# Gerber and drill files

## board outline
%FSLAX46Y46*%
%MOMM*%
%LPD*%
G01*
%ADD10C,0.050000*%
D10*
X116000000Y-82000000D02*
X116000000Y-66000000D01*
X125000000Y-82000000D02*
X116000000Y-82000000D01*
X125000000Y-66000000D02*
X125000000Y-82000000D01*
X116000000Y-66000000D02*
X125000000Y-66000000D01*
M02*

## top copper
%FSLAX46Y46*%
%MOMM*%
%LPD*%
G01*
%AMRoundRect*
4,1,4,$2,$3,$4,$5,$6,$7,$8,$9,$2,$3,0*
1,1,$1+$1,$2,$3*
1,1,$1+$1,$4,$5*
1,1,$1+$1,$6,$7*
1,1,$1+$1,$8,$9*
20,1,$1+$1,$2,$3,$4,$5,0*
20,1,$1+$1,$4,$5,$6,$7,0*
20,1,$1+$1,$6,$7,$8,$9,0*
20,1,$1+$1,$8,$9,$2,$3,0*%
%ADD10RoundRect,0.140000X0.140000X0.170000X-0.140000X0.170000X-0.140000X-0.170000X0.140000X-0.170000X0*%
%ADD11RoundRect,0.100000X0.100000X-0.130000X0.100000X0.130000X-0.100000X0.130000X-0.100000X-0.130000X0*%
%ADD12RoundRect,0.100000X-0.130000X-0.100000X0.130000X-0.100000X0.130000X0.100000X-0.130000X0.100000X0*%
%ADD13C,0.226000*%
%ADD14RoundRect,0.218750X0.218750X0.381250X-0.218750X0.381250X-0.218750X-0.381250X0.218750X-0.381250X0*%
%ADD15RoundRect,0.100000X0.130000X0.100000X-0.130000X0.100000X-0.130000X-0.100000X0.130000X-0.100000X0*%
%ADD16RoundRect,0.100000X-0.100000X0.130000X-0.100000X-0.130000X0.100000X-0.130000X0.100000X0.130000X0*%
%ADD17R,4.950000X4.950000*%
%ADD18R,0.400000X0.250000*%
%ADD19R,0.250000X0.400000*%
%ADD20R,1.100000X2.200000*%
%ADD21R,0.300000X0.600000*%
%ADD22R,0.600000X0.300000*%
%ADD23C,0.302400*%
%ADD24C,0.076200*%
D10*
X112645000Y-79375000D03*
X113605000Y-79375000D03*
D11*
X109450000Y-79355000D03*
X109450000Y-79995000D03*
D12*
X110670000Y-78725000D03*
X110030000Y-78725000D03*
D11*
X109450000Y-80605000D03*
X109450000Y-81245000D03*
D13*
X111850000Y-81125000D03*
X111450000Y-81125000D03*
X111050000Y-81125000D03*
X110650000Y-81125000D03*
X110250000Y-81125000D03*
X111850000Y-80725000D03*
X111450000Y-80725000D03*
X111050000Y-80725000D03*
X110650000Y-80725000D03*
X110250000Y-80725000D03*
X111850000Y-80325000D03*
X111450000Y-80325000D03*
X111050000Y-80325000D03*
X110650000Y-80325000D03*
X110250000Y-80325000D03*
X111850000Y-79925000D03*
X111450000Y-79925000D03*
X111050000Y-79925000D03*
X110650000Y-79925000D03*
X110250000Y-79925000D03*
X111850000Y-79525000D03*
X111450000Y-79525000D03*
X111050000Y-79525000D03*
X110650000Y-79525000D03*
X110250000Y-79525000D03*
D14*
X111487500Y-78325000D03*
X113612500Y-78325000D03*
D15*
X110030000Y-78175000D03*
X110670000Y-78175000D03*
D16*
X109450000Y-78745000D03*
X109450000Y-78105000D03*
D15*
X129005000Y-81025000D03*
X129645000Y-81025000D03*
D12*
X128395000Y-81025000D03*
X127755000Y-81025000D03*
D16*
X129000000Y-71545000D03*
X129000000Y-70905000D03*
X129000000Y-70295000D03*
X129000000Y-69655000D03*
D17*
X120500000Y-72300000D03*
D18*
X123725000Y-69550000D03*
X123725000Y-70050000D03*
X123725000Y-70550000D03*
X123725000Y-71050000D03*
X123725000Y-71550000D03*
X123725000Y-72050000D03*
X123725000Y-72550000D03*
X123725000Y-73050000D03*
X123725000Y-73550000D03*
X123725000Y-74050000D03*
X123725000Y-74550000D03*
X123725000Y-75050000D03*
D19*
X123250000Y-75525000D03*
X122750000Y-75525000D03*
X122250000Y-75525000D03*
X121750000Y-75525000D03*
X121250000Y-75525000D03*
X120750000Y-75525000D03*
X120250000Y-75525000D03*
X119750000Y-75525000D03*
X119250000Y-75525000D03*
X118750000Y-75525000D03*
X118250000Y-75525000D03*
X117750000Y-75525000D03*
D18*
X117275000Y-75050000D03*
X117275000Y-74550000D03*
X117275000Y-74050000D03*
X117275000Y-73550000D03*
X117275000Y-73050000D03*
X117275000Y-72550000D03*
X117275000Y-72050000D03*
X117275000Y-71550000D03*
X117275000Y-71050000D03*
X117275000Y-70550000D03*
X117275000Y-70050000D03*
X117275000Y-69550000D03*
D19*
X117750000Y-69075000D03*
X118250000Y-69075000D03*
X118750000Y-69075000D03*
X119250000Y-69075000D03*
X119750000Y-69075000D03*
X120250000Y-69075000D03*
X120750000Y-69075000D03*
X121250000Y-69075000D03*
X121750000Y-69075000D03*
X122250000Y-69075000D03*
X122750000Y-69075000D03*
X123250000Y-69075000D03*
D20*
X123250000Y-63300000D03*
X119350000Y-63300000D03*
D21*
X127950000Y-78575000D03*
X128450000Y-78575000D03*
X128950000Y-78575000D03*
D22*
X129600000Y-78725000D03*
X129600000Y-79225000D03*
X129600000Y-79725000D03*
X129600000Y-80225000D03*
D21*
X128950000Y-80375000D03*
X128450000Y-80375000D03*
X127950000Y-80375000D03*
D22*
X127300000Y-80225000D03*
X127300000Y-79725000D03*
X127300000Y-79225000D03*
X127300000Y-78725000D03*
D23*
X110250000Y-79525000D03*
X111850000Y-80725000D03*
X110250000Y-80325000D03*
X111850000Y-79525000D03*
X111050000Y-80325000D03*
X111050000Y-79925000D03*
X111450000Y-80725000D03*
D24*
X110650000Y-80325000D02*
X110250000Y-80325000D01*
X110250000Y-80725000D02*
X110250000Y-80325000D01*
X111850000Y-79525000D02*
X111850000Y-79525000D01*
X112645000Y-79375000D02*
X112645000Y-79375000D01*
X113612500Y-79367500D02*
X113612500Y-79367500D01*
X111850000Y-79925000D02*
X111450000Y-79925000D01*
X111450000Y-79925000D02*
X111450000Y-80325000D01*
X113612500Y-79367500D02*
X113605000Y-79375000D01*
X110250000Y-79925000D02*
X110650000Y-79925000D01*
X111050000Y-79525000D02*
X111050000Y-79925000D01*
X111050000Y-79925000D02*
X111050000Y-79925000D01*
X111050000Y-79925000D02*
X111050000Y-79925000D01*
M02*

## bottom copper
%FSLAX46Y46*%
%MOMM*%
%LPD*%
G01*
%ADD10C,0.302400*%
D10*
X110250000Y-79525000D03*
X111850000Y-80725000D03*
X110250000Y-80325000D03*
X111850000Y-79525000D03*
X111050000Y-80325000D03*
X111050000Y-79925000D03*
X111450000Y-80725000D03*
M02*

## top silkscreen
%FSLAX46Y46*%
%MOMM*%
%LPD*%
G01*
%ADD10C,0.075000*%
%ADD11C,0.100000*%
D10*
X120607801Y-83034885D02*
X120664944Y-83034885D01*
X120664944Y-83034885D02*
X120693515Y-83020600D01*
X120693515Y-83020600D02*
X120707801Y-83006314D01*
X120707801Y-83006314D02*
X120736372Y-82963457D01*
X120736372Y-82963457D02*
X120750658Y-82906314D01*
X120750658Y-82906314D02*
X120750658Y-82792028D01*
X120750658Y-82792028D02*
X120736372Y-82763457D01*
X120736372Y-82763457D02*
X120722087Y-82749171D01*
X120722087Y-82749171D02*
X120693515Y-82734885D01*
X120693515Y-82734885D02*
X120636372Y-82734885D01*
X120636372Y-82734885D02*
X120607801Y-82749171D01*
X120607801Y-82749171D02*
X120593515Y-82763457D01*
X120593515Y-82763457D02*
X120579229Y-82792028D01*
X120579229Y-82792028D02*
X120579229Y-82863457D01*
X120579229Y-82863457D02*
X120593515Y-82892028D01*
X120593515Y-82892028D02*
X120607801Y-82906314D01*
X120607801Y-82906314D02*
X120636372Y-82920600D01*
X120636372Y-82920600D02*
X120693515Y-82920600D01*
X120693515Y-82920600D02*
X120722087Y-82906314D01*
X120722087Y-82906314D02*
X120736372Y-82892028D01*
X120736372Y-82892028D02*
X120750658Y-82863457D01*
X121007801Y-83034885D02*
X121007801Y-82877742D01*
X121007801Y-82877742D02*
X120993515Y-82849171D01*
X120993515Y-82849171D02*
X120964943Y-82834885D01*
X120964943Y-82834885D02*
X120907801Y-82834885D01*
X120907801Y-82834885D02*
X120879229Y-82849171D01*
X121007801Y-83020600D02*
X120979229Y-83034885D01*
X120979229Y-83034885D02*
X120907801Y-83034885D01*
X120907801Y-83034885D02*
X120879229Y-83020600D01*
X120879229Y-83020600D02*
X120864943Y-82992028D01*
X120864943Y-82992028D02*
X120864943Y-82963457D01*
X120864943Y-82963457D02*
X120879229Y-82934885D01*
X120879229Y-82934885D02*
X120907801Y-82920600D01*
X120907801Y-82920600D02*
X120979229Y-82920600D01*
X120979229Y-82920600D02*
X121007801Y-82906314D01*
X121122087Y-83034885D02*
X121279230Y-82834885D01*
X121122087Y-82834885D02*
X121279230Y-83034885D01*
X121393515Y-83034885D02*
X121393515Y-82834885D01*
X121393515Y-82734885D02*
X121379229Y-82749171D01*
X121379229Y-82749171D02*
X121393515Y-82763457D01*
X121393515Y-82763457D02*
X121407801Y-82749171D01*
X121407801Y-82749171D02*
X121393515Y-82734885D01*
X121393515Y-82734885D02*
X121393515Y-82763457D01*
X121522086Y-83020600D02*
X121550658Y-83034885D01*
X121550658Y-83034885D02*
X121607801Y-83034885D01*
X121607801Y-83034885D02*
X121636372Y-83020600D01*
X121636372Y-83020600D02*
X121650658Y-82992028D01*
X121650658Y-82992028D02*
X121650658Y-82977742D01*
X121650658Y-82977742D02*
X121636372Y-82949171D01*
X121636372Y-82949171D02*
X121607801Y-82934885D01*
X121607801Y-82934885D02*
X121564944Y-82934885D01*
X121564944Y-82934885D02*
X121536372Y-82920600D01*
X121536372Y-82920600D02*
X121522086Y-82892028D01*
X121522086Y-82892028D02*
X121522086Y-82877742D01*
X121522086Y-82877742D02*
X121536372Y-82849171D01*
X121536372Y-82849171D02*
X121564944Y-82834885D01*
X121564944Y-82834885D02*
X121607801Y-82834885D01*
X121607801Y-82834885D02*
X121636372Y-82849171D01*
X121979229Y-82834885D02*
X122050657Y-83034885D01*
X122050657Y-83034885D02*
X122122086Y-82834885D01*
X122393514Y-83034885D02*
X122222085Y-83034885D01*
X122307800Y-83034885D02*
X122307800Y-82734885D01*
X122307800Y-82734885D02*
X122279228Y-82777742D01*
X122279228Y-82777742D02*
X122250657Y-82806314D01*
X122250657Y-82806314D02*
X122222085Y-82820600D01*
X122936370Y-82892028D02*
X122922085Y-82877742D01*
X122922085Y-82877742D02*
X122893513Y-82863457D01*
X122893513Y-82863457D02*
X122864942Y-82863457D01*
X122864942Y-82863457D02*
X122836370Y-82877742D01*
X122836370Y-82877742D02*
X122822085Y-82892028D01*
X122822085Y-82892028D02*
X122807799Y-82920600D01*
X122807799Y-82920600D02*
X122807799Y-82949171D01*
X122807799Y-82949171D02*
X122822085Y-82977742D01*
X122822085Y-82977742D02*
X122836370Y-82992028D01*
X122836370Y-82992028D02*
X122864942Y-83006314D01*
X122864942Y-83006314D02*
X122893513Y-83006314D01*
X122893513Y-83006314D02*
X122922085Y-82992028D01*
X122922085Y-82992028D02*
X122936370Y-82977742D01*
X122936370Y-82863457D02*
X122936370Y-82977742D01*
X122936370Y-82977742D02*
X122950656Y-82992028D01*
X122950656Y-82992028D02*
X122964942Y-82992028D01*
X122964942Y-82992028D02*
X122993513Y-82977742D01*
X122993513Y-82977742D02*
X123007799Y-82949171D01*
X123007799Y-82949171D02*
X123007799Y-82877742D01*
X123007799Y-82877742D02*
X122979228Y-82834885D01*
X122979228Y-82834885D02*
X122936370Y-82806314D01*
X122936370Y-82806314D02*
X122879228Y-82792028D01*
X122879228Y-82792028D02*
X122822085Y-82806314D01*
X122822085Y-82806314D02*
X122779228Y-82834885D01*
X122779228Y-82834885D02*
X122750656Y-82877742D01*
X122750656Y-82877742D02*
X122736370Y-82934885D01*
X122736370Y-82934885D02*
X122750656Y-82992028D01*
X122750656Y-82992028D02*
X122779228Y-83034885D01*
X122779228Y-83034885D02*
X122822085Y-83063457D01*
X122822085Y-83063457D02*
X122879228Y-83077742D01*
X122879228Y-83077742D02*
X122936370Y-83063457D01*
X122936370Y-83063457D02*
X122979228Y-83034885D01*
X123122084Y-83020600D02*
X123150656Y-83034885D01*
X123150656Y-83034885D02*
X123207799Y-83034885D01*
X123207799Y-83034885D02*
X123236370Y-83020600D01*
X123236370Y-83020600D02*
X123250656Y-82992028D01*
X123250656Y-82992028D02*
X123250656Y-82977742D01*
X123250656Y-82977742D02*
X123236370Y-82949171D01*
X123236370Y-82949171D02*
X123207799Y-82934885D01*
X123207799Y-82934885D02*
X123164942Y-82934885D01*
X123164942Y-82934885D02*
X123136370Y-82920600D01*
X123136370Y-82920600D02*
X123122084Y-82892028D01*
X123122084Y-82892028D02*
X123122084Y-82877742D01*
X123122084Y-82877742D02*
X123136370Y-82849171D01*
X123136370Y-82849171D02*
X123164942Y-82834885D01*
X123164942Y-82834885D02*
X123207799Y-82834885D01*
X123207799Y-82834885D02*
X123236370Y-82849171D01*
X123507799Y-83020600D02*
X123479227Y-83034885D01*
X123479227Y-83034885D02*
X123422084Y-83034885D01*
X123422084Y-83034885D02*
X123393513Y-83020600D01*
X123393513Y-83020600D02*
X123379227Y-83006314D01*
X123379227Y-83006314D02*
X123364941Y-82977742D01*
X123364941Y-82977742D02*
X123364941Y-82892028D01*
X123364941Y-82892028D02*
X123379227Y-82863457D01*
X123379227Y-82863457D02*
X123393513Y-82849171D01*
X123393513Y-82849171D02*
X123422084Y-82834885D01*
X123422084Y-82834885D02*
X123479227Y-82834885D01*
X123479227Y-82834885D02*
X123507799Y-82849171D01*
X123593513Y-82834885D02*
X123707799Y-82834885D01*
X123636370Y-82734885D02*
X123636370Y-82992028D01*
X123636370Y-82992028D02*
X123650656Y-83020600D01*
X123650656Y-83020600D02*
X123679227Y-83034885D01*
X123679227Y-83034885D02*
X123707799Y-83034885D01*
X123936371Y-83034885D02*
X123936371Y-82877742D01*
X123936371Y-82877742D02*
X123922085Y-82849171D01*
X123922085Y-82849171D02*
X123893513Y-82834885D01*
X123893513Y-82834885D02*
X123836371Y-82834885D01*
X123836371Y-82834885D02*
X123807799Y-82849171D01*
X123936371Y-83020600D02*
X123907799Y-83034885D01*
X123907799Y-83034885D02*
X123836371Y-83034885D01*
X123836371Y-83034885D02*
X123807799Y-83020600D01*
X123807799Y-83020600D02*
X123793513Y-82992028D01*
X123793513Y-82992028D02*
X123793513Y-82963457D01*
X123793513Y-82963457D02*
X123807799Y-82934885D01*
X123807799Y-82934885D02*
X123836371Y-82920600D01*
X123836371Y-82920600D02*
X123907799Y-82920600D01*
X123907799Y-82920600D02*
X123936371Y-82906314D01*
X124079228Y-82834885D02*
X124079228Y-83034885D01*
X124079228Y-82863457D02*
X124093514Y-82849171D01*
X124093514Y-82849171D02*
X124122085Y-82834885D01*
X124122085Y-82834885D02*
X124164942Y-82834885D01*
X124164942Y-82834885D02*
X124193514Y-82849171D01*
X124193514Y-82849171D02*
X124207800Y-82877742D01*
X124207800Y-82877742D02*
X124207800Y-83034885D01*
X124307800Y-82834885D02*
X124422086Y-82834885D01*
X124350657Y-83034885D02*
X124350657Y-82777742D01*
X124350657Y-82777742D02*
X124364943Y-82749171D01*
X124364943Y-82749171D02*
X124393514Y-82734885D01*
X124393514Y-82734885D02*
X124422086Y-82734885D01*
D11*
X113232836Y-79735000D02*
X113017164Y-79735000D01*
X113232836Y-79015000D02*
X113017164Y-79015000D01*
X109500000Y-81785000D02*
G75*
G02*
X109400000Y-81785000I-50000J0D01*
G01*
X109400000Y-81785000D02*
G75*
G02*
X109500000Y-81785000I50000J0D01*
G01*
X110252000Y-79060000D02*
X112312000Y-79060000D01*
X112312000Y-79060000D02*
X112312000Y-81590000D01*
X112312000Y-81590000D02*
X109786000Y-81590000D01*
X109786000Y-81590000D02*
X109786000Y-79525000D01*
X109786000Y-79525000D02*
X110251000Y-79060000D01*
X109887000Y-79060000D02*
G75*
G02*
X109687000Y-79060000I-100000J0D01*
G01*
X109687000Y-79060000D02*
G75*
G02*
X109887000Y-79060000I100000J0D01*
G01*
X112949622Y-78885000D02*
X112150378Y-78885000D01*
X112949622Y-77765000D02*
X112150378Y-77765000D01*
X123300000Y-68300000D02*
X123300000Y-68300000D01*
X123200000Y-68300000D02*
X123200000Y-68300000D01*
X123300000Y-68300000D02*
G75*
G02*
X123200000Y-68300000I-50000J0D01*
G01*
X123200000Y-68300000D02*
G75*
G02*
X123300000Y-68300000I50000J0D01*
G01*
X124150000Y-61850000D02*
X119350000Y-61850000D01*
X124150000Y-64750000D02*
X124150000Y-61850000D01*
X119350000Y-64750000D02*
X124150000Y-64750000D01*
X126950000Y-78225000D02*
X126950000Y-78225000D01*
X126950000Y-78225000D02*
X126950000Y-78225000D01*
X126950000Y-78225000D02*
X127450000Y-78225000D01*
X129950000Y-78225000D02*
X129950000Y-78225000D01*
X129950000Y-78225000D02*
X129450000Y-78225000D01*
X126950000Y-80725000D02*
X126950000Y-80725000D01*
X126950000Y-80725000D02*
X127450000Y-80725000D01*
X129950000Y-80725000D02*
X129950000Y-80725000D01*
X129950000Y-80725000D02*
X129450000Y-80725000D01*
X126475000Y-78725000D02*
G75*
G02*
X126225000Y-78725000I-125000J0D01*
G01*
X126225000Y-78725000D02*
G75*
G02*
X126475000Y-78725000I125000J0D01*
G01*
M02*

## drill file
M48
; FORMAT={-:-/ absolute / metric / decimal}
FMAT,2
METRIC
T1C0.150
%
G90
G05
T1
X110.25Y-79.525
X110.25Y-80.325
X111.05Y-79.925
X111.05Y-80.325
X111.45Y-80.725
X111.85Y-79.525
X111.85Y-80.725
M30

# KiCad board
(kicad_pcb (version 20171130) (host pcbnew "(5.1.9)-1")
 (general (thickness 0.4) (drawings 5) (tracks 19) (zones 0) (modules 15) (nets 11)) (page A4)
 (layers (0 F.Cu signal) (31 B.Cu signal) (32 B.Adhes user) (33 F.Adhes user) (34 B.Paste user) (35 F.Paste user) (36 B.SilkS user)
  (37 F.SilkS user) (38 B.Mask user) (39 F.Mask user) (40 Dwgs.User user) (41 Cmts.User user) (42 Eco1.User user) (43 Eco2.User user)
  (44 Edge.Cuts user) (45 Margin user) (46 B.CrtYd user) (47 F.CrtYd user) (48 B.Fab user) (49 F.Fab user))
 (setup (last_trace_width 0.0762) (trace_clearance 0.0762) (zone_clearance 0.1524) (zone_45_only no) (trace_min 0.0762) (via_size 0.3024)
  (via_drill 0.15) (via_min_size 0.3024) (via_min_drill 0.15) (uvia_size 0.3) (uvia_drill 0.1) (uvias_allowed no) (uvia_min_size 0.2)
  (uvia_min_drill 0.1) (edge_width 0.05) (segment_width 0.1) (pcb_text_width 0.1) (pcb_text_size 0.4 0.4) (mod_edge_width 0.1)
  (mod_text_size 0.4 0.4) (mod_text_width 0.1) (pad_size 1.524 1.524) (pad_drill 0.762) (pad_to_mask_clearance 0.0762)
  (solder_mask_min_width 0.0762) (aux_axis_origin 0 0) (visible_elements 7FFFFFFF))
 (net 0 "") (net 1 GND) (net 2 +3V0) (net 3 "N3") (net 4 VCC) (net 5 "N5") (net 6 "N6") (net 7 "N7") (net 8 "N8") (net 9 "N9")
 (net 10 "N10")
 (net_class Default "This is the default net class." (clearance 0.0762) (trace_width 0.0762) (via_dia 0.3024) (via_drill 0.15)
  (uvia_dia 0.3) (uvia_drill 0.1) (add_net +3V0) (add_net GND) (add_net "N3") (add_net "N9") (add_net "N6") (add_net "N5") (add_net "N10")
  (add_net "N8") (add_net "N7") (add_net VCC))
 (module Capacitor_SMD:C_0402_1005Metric (layer F.Cu) (at 113.125 79.375 180)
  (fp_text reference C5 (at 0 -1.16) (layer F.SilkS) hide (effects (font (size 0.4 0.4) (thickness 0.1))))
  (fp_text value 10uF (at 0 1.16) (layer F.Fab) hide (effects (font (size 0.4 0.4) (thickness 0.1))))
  (fp_line (start -0.107836 -0.36) (end 0.107836 -0.36) (layer F.SilkS) (width 0.1))
  (fp_line (start -0.107836 0.36) (end 0.107836 0.36) (layer F.SilkS) (width 0.1))
  (pad 2 smd roundrect (at 0.48 0 180) (size 0.56 0.62) (layers F.Cu F.Paste F.Mask) (roundrect_rratio 0.25) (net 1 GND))
  (pad 1 smd roundrect (at -0.48 0 180) (size 0.56 0.62) (layers F.Cu F.Paste F.Mask) (roundrect_rratio 0.25) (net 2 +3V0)))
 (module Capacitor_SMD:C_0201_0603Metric (layer F.Cu) (at 109.45 79.675 90)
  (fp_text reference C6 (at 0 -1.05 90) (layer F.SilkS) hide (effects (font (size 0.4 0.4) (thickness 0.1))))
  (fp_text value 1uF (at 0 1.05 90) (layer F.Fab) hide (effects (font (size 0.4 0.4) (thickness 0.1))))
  (pad 2 smd roundrect (at 0.32 0 90) (size 0.46 0.4) (layers F.Cu F.Mask) (roundrect_rratio 0.25) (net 1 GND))
  (pad 1 smd roundrect (at -0.32 0 90) (size 0.46 0.4) (layers F.Cu F.Mask) (roundrect_rratio 0.25) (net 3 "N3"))
  (pad "" smd roundrect (at 0.345 0 90) (size 0.318 0.36) (layers F.Paste) (roundrect_rratio 0.25))
  (pad "" smd roundrect (at -0.345 0 90) (size 0.318 0.36) (layers F.Paste) (roundrect_rratio 0.25)))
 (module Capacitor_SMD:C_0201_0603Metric (layer F.Cu) (at 110.35 78.725)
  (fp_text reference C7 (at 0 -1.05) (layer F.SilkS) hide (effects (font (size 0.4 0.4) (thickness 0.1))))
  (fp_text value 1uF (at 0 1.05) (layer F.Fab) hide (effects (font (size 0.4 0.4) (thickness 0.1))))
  (pad 2 smd roundrect (at 0.32 0) (size 0.46 0.4) (layers F.Cu F.Mask) (roundrect_rratio 0.25) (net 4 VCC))
  (pad 1 smd roundrect (at -0.32 0) (size 0.46 0.4) (layers F.Cu F.Mask) (roundrect_rratio 0.25) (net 1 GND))
  (pad "" smd roundrect (at 0.345 0) (size 0.318 0.36) (layers F.Paste) (roundrect_rratio 0.25))
  (pad "" smd roundrect (at -0.345 0) (size 0.318 0.36) (layers F.Paste) (roundrect_rratio 0.25)))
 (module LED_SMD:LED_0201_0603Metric (layer F.Cu) (at 109.45 80.925 90)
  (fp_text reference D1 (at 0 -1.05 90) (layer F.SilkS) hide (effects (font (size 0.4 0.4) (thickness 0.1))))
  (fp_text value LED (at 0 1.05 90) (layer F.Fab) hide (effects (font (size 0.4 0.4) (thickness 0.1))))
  (fp_circle (center -0.86 0) (end -0.81 0) (layer F.SilkS) (width 0.1))
  (pad 2 smd roundrect (at 0.32 0 90) (size 0.46 0.4) (layers F.Cu F.Mask) (roundrect_rratio 0.25) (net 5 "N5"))
  (pad 1 smd roundrect (at -0.32 0 90) (size 0.46 0.4) (layers F.Cu F.Mask) (roundrect_rratio 0.25) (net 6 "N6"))
  (pad "" smd roundrect (at 0.345 0 90) (size 0.318 0.36) (layers F.Paste) (roundrect_rratio 0.25))
  (pad "" smd roundrect (at -0.345 0 90) (size 0.318 0.36) (layers F.Paste) (roundrect_rratio 0.25)))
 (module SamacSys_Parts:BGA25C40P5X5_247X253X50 (layer F.Cu) (at 111.05 80.325)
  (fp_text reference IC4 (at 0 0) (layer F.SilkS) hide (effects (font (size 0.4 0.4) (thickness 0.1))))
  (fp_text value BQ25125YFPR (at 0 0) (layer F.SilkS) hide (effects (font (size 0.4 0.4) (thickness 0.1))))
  (fp_line (start -0.798 -1.265) (end 1.262 -1.265) (layer F.SilkS) (width 0.1))
  (fp_line (start 1.262 -1.265) (end 1.262 1.265) (layer F.SilkS) (width 0.1))
  (fp_line (start 1.262 1.265) (end -1.264 1.265) (layer F.SilkS) (width 0.1))
  (fp_line (start -1.264 1.265) (end -1.264 -0.8) (layer F.SilkS) (width 0.1))
  (fp_line (start -1.264 -0.8) (end -0.799 -1.265) (layer F.SilkS) (width 0.1))
  (fp_circle (center -1.263 -1.265) (end -1.263 -1.165) (layer F.SilkS) (width 0.1))
  (pad E5 smd circle (at 0.8 0.8 90) (size 0.226 0.226) (layers F.Cu F.Paste F.Mask))
  (pad E4 smd circle (at 0.4 0.8 90) (size 0.226 0.226) (layers F.Cu F.Paste F.Mask))
  (pad E3 smd circle (at 0 0.8 90) (size 0.226 0.226) (layers F.Cu F.Paste F.Mask))
  (pad E2 smd circle (at -0.4 0.8 90) (size 0.226 0.226) (layers F.Cu F.Paste F.Mask))
  (pad E1 smd circle (at -0.8 0.8 90) (size 0.226 0.226) (layers F.Cu F.Paste F.Mask))
  (pad D5 smd circle (at 0.8 0.4 90) (size 0.226 0.226) (layers F.Cu F.Paste F.Mask) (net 1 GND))
  (pad D4 smd circle (at 0.4 0.4 90) (size 0.226 0.226) (layers F.Cu F.Paste F.Mask) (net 6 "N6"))
  (pad D3 smd circle (at 0 0.4 90) (size 0.226 0.226) (layers F.Cu F.Paste F.Mask))
  (pad D2 smd circle (at -0.4 0.4 90) (size 0.226 0.226) (layers F.Cu F.Paste F.Mask))
  (pad D1 smd circle (at -0.8 0.4 90) (size 0.226 0.226) (layers F.Cu F.Paste F.Mask) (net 1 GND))
  (pad C5 smd circle (at 0.8 0 90) (size 0.226 0.226) (layers F.Cu F.Paste F.Mask))
  (pad C4 smd circle (at 0.4 0 90) (size 0.226 0.226) (layers F.Cu F.Paste F.Mask) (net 2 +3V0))
  (pad C3 smd circle (at 0 0 90) (size 0.226 0.226) (layers F.Cu F.Paste F.Mask) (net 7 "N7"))
  (pad C2 smd circle (at -0.4 0 90) (size 0.226 0.226) (layers F.Cu F.Paste F.Mask) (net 1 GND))
  (pad C1 smd circle (at -0.8 0 90) (size 0.226 0.226) (layers F.Cu F.Paste F.Mask) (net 1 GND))
  (pad B5 smd circle (at 0.8 -0.4 90) (size 0.226 0.226) (layers F.Cu F.Paste F.Mask) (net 2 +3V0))
  (pad B4 smd circle (at 0.4 -0.4 90) (size 0.226 0.226) (layers F.Cu F.Paste F.Mask) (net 2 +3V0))
  (pad B3 smd circle (at 0 -0.4 90) (size 0.226 0.226) (layers F.Cu F.Paste F.Mask) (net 5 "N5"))
  (pad B2 smd circle (at -0.4 -0.4 90) (size 0.226 0.226) (layers F.Cu F.Paste F.Mask) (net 3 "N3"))
  (pad B1 smd circle (at -0.8 -0.4 90) (size 0.226 0.226) (layers F.Cu F.Paste F.Mask) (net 3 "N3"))
  (pad A5 smd circle (at 0.8 -0.8 90) (size 0.226 0.226) (layers F.Cu F.Paste F.Mask) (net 1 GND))
  (pad A4 smd circle (at 0.4 -0.8 90) (size 0.226 0.226) (layers F.Cu F.Paste F.Mask) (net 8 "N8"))
  (pad A3 smd circle (at 0 -0.8 90) (size 0.226 0.226) (layers F.Cu F.Paste F.Mask) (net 5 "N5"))
  (pad A2 smd circle (at -0.4 -0.8 90) (size 0.226 0.226) (layers F.Cu F.Paste F.Mask) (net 4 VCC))
  (pad A1 smd circle (at -0.8 -0.8 90) (size 0.226 0.226) (layers F.Cu F.Paste F.Mask) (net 1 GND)))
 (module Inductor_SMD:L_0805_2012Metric (layer F.Cu) (at 112.55 78.325 180)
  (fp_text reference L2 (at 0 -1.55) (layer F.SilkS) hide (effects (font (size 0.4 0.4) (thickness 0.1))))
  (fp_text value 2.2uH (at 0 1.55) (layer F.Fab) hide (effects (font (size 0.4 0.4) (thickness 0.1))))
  (fp_line (start -0.399622 -0.56) (end 0.399622 -0.56) (layer F.SilkS) (width 0.1))
  (fp_line (start -0.399622 0.56) (end 0.399622 0.56) (layer F.SilkS) (width 0.1))
  (pad 2 smd roundrect (at 1.0625 0 180) (size 0.875 1.2) (layers F.Cu F.Paste F.Mask) (roundrect_rratio 0.25) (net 8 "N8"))
  (pad 1 smd roundrect (at -1.0625 0 180) (size 0.875 1.2) (layers F.Cu F.Paste F.Mask) (roundrect_rratio 0.25) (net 2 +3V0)))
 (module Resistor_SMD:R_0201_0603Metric (layer F.Cu) (at 110.35 78.175 180)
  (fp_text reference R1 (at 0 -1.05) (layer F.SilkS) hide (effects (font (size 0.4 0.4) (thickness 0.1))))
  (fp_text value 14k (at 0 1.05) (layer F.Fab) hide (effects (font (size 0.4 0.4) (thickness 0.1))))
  (pad 2 smd roundrect (at 0.32 0 180) (size 0.46 0.4) (layers F.Cu F.Mask) (roundrect_rratio 0.25) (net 7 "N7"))
  (pad 1 smd roundrect (at -0.32 0 180) (size 0.46 0.4) (layers F.Cu F.Mask) (roundrect_rratio 0.25) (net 4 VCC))
  (pad "" smd roundrect (at 0.345 0 180) (size 0.318 0.36) (layers F.Paste) (roundrect_rratio 0.25))
  (pad "" smd roundrect (at -0.345 0 180) (size 0.318 0.36) (layers F.Paste) (roundrect_rratio 0.25)))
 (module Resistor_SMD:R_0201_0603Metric (layer F.Cu) (at 109.45 78.425 270)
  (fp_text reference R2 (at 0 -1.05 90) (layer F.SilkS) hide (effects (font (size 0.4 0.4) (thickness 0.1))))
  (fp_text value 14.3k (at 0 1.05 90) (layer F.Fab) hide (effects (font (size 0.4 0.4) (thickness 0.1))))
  (pad 2 smd roundrect (at 0.32 0 270) (size 0.46 0.4) (layers F.Cu F.Mask) (roundrect_rratio 0.25) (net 1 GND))
  (pad 1 smd roundrect (at -0.32 0 270) (size 0.46 0.4) (layers F.Cu F.Mask) (roundrect_rratio 0.25) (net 7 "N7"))
  (pad "" smd roundrect (at 0.345 0 270) (size 0.318 0.36) (layers F.Paste) (roundrect_rratio 0.25))
  (pad "" smd roundrect (at -0.345 0 270) (size 0.318 0.36) (layers F.Paste) (roundrect_rratio 0.25)))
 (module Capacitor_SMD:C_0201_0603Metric (layer F.Cu) (at 129.325 81.025 180)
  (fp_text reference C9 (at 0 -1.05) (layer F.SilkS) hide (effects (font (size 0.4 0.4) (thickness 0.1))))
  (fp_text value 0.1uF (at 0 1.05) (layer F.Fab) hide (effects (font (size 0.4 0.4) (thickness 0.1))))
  (pad 2 smd roundrect (at 0.32 0 180) (size 0.46 0.4) (layers F.Cu F.Mask) (roundrect_rratio 0.25) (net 1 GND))
  (pad 1 smd roundrect (at -0.32 0 180) (size 0.46 0.4) (layers F.Cu F.Mask) (roundrect_rratio 0.25) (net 2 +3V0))
  (pad "" smd roundrect (at 0.345 0 180) (size 0.318 0.36) (layers F.Paste) (roundrect_rratio 0.25))
  (pad "" smd roundrect (at -0.345 0 180) (size 0.318 0.36) (layers F.Paste) (roundrect_rratio 0.25)))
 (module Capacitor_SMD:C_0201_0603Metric (layer F.Cu) (at 128.075 81.025)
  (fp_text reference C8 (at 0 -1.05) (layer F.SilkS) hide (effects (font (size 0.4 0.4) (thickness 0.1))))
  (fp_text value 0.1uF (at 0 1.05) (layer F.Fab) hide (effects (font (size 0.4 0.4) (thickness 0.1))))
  (pad 2 smd roundrect (at 0.32 0) (size 0.46 0.4) (layers F.Cu F.Mask) (roundrect_rratio 0.25) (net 1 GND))
  (pad 1 smd roundrect (at -0.32 0) (size 0.46 0.4) (layers F.Cu F.Mask) (roundrect_rratio 0.25) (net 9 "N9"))
  (pad "" smd roundrect (at 0.345 0) (size 0.318 0.36) (layers F.Paste) (roundrect_rratio 0.25))
  (pad "" smd roundrect (at -0.345 0) (size 0.318 0.36) (layers F.Paste) (roundrect_rratio 0.25)))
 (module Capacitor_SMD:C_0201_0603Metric (layer F.Cu) (at 129 71.225 270)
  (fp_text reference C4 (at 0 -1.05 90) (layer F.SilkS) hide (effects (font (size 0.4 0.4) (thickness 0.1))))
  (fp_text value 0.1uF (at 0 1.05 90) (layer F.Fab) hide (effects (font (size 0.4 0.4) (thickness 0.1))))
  (pad 2 smd roundrect (at 0.32 0 270) (size 0.46 0.4) (layers F.Cu F.Mask) (roundrect_rratio 0.25) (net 1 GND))
  (pad 1 smd roundrect (at -0.32 0 270) (size 0.46 0.4) (layers F.Cu F.Mask) (roundrect_rratio 0.25) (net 2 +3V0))
  (pad "" smd roundrect (at 0.345 0 270) (size 0.318 0.36) (layers F.Paste) (roundrect_rratio 0.25))
  (pad "" smd roundrect (at -0.345 0 270) (size 0.318 0.36) (layers F.Paste) (roundrect_rratio 0.25)))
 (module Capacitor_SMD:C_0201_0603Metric (layer F.Cu) (at 129 69.975 270)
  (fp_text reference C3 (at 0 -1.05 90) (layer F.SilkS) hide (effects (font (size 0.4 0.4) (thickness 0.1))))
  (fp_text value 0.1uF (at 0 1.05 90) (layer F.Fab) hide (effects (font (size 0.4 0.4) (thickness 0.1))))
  (pad 2 smd roundrect (at 0.32 0 270) (size 0.46 0.4) (layers F.Cu F.Mask) (roundrect_rratio 0.25) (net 1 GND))
  (pad 1 smd roundrect (at -0.32 0 270) (size 0.46 0.4) (layers F.Cu F.Mask) (roundrect_rratio 0.25) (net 2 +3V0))
  (pad "" smd roundrect (at 0.345 0 270) (size 0.318 0.36) (layers F.Paste) (roundrect_rratio 0.25))
  (pad "" smd roundrect (at -0.345 0 270) (size 0.318 0.36) (layers F.Paste) (roundrect_rratio 0.25)))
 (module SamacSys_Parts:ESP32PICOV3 (layer F.Cu) (at 120.5 72.3 270)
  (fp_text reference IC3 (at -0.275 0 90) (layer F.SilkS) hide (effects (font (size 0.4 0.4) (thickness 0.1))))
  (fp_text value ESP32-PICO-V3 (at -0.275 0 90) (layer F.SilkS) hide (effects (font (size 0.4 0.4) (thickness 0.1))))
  (fp_line (start -4 -2.8) (end -4 -2.8) (layer F.SilkS) (width 0.1))
  (fp_line (start -4 -2.7) (end -4 -2.7) (layer F.SilkS) (width 0.1))
  (fp_arc (start -4 -2.75) (end -4 -2.7) (angle -180) (layer F.SilkS) (width 0.1))
  (fp_arc (start -4 -2.75) (end -4 -2.8) (angle -180) (layer F.SilkS) (width 0.1))
  (pad 49 smd rect (at 0 0 270) (size 4.95 4.95) (layers F.Cu F.Paste F.Mask) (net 1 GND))
  (pad 48 smd rect (at -2.75 -3.225 270) (size 0.25 0.4) (layers F.Cu F.Paste F.Mask))
  (pad 47 smd rect (at -2.25 -3.225 270) (size 0.25 0.4) (layers F.Cu F.Paste F.Mask))
  (pad 46 smd rect (at -1.75 -3.225 270) (size 0.25 0.4) (layers F.Cu F.Paste F.Mask) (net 2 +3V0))
  (pad 45 smd rect (at -1.25 -3.225 270) (size 0.25 0.4) (layers F.Cu F.Paste F.Mask))
  (pad 44 smd rect (at -0.75 -3.225 270) (size 0.25 0.4) (layers F.Cu F.Paste F.Mask))
  (pad 43 smd rect (at -0.25 -3.225 270) (size 0.25 0.4) (layers F.Cu F.Paste F.Mask) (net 2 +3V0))
  (pad 42 smd rect (at 0.25 -3.225 270) (size 0.25 0.4) (layers F.Cu F.Paste F.Mask))
  (pad 41 smd rect (at 0.75 -3.225 270) (size 0.25 0.4) (layers F.Cu F.Paste F.Mask))
  (pad 40 smd rect (at 1.25 -3.225 270) (size 0.25 0.4) (layers F.Cu F.Paste F.Mask))
  (pad 39 smd rect (at 1.75 -3.225 270) (size 0.25 0.4) (layers F.Cu F.Paste F.Mask))
  (pad 38 smd rect (at 2.25 -3.225 270) (size 0.25 0.4) (layers F.Cu F.Paste F.Mask))
  (pad 37 smd rect (at 2.75 -3.225 270) (size 0.25 0.4) (layers F.Cu F.Paste F.Mask) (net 2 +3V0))
  (pad 36 smd rect (at 3.225 -2.75) (size 0.25 0.4) (layers F.Cu F.Paste F.Mask))
  (pad 35 smd rect (at 3.225 -2.25) (size 0.25 0.4) (layers F.Cu F.Paste F.Mask))
  (pad 34 smd rect (at 3.225 -1.75) (size 0.25 0.4) (layers F.Cu F.Paste F.Mask))
  (pad 33 smd rect (at 3.225 -1.25) (size 0.25 0.4) (layers F.Cu F.Paste F.Mask))
  (pad 32 smd rect (at 3.225 -0.75) (size 0.25 0.4) (layers F.Cu F.Paste F.Mask))
  (pad 31 smd rect (at 3.225 -0.25) (size 0.25 0.4) (layers F.Cu F.Paste F.Mask))
  (pad 30 smd rect (at 3.225 0.25) (size 0.25 0.4) (layers F.Cu F.Paste F.Mask))
  (pad 29 smd rect (at 3.225 0.75) (size 0.25 0.4) (layers F.Cu F.Paste F.Mask))
  (pad 28 smd rect (at 3.225 1.25) (size 0.25 0.4) (layers F.Cu F.Paste F.Mask))
  (pad 27 smd rect (at 3.225 1.75) (size 0.25 0.4) (layers F.Cu F.Paste F.Mask))
  (pad 26 smd rect (at 3.225 2.25) (size 0.25 0.4) (layers F.Cu F.Paste F.Mask))
  (pad 25 smd rect (at 3.225 2.75) (size 0.25 0.4) (layers F.Cu F.Paste F.Mask))
  (pad 24 smd rect (at 2.75 3.225 270) (size 0.25 0.4) (layers F.Cu F.Paste F.Mask))
  (pad 23 smd rect (at 2.25 3.225 270) (size 0.25 0.4) (layers F.Cu F.Paste F.Mask))
  (pad 22 smd rect (at 1.75 3.225 270) (size 0.25 0.4) (layers F.Cu F.Paste F.Mask))
  (pad 21 smd rect (at 1.25 3.225 270) (size 0.25 0.4) (layers F.Cu F.Paste F.Mask))
  (pad 20 smd rect (at 0.75 3.225 270) (size 0.25 0.4) (layers F.Cu F.Paste F.Mask))
  (pad 19 smd rect (at 0.25 3.225 270) (size 0.25 0.4) (layers F.Cu F.Paste F.Mask) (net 2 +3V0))
  (pad 18 smd rect (at -0.25 3.225 270) (size 0.25 0.4) (layers F.Cu F.Paste F.Mask))
  (pad 17 smd rect (at -0.75 3.225 270) (size 0.25 0.4) (layers F.Cu F.Paste F.Mask))
  (pad 16 smd rect (at -1.25 3.225 270) (size 0.25 0.4) (layers F.Cu F.Paste F.Mask))
  (pad 15 smd rect (at -1.75 3.225 270) (size 0.25 0.4) (layers F.Cu F.Paste F.Mask))
  (pad 14 smd rect (at -2.25 3.225 270) (size 0.25 0.4) (layers F.Cu F.Paste F.Mask))
  (pad 13 smd rect (at -2.75 3.225 270) (size 0.25 0.4) (layers F.Cu F.Paste F.Mask))
  (pad 12 smd rect (at -3.225 2.75) (size 0.25 0.4) (layers F.Cu F.Paste F.Mask))
  (pad 11 smd rect (at -3.225 2.25) (size 0.25 0.4) (layers F.Cu F.Paste F.Mask))
  (pad 10 smd rect (at -3.225 1.75) (size 0.25 0.4) (layers F.Cu F.Paste F.Mask))
  (pad 9 smd rect (at -3.225 1.25) (size 0.25 0.4) (layers F.Cu F.Paste F.Mask))
  (pad 8 smd rect (at -3.225 0.75) (size 0.25 0.4) (layers F.Cu F.Paste F.Mask))
  (pad 7 smd rect (at -3.225 0.25) (size 0.25 0.4) (layers F.Cu F.Paste F.Mask))
  (pad 6 smd rect (at -3.225 -0.25) (size 0.25 0.4) (layers F.Cu F.Paste F.Mask))
  (pad 5 smd rect (at -3.225 -0.75) (size 0.25 0.4) (layers F.Cu F.Paste F.Mask))
  (pad 4 smd rect (at -3.225 -1.25) (size 0.25 0.4) (layers F.Cu F.Paste F.Mask) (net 2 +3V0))
  (pad 3 smd rect (at -3.225 -1.75) (size 0.25 0.4) (layers F.Cu F.Paste F.Mask) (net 2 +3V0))
  (pad 2 smd rect (at -3.225 -2.25) (size 0.25 0.4) (layers F.Cu F.Paste F.Mask) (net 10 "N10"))
  (pad 1 smd rect (at -3.225 -2.75) (size 0.25 0.4) (layers F.Cu F.Paste F.Mask) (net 2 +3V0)))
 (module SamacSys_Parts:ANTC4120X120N (layer F.Cu) (at 121.3 63.3 180)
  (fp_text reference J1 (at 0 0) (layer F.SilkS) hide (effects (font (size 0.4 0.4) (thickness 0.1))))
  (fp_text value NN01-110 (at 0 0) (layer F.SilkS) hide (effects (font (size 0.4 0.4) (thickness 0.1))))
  (fp_line (start -2.85 1.45) (end 1.95 1.45) (layer F.SilkS) (width 0.1))
  (fp_line (start -2.85 -1.45) (end -2.85 1.45) (layer F.SilkS) (width 0.1))
  (fp_line (start 1.95 -1.45) (end -2.85 -1.45) (layer F.SilkS) (width 0.1))
  (pad 1 smd rect (at -1.95 0 180) (size 1.1 2.2) (layers F.Cu F.Paste F.Mask) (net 10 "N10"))
  (pad 2 smd rect (at 1.95 0 180) (size 1.1 2.2) (layers F.Cu F.Paste F.Mask)))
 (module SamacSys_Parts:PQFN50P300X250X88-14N (layer F.Cu) (at 128.45 79.475)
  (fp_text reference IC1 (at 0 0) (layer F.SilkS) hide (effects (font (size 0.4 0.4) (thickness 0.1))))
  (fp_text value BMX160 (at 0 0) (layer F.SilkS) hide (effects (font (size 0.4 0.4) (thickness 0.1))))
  (fp_line (start -1.5 -1.25) (end -1.5 -1.25) (layer F.SilkS) (width 0.1))
  (fp_line (start -1.5 -1.25) (end -1.5 -1.25) (layer F.SilkS) (width 0.1))
  (fp_line (start -1.5 -1.25) (end -1 -1.25) (layer F.SilkS) (width 0.1))
  (fp_line (start 1.5 -1.25) (end 1.5 -1.25) (layer F.SilkS) (width 0.1))
  (fp_line (start 1.5 -1.25) (end 1 -1.25) (layer F.SilkS) (width 0.1))
  (fp_line (start -1.5 1.25) (end -1.5 1.25) (layer F.SilkS) (width 0.1))
  (fp_line (start -1.5 1.25) (end -1 1.25) (layer F.SilkS) (width 0.1))
  (fp_line (start 1.5 1.25) (end 1.5 1.25) (layer F.SilkS) (width 0.1))
  (fp_line (start 1.5 1.25) (end 1 1.25) (layer F.SilkS) (width 0.1))
  (fp_circle (center -2.1 -0.75) (end -2.1 -0.625) (layer F.SilkS) (width 0.1))
  (pad 14 smd rect (at -0.5 -0.9) (size 0.3 0.6) (layers F.Cu F.Paste F.Mask))
  (pad 13 smd rect (at 0 -0.9) (size 0.3 0.6) (layers F.Cu F.Paste F.Mask))
  (pad 12 smd rect (at 0.5 -0.9) (size 0.3 0.6) (layers F.Cu F.Paste F.Mask))
  (pad 11 smd rect (at 1.15 -0.75 90) (size 0.3 0.6) (layers F.Cu F.Paste F.Mask))
  (pad 10 smd rect (at 1.15 -0.25 90) (size 0.3 0.6) (layers F.Cu F.Paste F.Mask))
  (pad 9 smd rect (at 1.15 0.25 90) (size 0.3 0.6) (layers F.Cu F.Paste F.Mask))
  (pad 8 smd rect (at 1.15 0.75 90) (size 0.3 0.6) (layers F.Cu F.Paste F.Mask) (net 2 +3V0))
  (pad 7 smd rect (at 0.5 0.9) (size 0.3 0.6) (layers F.Cu F.Paste F.Mask) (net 1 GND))
  (pad 6 smd rect (at 0 0.9) (size 0.3 0.6) (layers F.Cu F.Paste F.Mask) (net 1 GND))
  (pad 5 smd rect (at -0.5 0.9) (size 0.3 0.6) (layers F.Cu F.Paste F.Mask) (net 9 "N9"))
  (pad 4 smd rect (at -1.15 0.75 90) (size 0.3 0.6) (layers F.Cu F.Paste F.Mask))
  (pad 3 smd rect (at -1.15 0.25 90) (size 0.3 0.6) (layers F.Cu F.Paste F.Mask) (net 1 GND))
  (pad 2 smd rect (at -1.15 -0.25 90) (size 0.3 0.6) (layers F.Cu F.Paste F.Mask) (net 1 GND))
  (pad 1 smd rect (at -1.15 -0.75 90) (size 0.3 0.6) (layers F.Cu F.Paste F.Mask)))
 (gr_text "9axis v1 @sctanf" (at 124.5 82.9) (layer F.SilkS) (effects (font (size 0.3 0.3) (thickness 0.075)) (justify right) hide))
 (gr_line (start 116 82) (end 116 66) (layer Edge.Cuts) (width 0.05))
 (gr_line (start 125 82) (end 116 82) (layer Edge.Cuts) (width 0.05))
 (gr_line (start 125 66) (end 125 82) (layer Edge.Cuts) (width 0.05))
 (gr_line (start 116 66) (end 125 66) (layer Edge.Cuts) (width 0.05))
 (via (at 110.25 79.525) (size 0.3024) (drill 0.15) (layers F.Cu B.Cu) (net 1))
 (via (at 111.85 80.725) (size 0.3024) (drill 0.15) (layers F.Cu B.Cu) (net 1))
 (segment (start 110.65 80.325) (end 110.25 80.325) (width 0.0762) (layer F.Cu) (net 1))
 (segment (start 110.25 80.725) (end 110.25 80.325) (width 0.0762) (layer F.Cu) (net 1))
 (via (at 110.25 80.325) (size 0.3024) (drill 0.15) (layers F.Cu B.Cu) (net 1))
 (via (at 111.85 79.525) (size 0.3024) (drill 0.15) (layers F.Cu B.Cu) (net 1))
 (segment (start 111.85 79.525) (end 111.85 79.525) (width 0.0762) (layer F.Cu) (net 1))
 (segment (start 112.645 79.375) (end 112.645 79.375) (width 0.0762) (layer F.Cu) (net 1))
 (segment (start 113.6125 79.3675) (end 113.6125 79.3675) (width 0.0762) (layer F.Cu) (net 2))
 (segment (start 111.85 79.925) (end 111.45 79.925) (width 0.0762) (layer F.Cu) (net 2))
 (segment (start 111.45 79.925) (end 111.45 80.325) (width 0.0762) (layer F.Cu) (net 2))
 (segment (start 113.6125 79.3675) (end 113.605 79.375) (width 0.0762) (layer F.Cu) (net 2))
 (via (at 111.05 80.325) (size 0.3024) (drill 0.15) (layers F.Cu B.Cu) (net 7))
 (segment (start 110.25 79.925) (end 110.65 79.925) (width 0.0762) (layer F.Cu) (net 3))
 (segment (start 111.05 79.525) (end 111.05 79.925) (width 0.0762) (layer F.Cu) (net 5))
 (segment (start 111.05 79.925) (end 111.05 79.925) (width 0.0762) (layer F.Cu) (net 5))
 (segment (start 111.05 79.925) (end 111.05 79.925) (width 0.0762) (layer F.Cu) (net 5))
 (via (at 111.05 79.925) (size 0.3024) (drill 0.15) (layers F.Cu B.Cu) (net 5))
 (via (at 111.45 80.725) (size 0.3024) (drill 0.15) (layers F.Cu B.Cu) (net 6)))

